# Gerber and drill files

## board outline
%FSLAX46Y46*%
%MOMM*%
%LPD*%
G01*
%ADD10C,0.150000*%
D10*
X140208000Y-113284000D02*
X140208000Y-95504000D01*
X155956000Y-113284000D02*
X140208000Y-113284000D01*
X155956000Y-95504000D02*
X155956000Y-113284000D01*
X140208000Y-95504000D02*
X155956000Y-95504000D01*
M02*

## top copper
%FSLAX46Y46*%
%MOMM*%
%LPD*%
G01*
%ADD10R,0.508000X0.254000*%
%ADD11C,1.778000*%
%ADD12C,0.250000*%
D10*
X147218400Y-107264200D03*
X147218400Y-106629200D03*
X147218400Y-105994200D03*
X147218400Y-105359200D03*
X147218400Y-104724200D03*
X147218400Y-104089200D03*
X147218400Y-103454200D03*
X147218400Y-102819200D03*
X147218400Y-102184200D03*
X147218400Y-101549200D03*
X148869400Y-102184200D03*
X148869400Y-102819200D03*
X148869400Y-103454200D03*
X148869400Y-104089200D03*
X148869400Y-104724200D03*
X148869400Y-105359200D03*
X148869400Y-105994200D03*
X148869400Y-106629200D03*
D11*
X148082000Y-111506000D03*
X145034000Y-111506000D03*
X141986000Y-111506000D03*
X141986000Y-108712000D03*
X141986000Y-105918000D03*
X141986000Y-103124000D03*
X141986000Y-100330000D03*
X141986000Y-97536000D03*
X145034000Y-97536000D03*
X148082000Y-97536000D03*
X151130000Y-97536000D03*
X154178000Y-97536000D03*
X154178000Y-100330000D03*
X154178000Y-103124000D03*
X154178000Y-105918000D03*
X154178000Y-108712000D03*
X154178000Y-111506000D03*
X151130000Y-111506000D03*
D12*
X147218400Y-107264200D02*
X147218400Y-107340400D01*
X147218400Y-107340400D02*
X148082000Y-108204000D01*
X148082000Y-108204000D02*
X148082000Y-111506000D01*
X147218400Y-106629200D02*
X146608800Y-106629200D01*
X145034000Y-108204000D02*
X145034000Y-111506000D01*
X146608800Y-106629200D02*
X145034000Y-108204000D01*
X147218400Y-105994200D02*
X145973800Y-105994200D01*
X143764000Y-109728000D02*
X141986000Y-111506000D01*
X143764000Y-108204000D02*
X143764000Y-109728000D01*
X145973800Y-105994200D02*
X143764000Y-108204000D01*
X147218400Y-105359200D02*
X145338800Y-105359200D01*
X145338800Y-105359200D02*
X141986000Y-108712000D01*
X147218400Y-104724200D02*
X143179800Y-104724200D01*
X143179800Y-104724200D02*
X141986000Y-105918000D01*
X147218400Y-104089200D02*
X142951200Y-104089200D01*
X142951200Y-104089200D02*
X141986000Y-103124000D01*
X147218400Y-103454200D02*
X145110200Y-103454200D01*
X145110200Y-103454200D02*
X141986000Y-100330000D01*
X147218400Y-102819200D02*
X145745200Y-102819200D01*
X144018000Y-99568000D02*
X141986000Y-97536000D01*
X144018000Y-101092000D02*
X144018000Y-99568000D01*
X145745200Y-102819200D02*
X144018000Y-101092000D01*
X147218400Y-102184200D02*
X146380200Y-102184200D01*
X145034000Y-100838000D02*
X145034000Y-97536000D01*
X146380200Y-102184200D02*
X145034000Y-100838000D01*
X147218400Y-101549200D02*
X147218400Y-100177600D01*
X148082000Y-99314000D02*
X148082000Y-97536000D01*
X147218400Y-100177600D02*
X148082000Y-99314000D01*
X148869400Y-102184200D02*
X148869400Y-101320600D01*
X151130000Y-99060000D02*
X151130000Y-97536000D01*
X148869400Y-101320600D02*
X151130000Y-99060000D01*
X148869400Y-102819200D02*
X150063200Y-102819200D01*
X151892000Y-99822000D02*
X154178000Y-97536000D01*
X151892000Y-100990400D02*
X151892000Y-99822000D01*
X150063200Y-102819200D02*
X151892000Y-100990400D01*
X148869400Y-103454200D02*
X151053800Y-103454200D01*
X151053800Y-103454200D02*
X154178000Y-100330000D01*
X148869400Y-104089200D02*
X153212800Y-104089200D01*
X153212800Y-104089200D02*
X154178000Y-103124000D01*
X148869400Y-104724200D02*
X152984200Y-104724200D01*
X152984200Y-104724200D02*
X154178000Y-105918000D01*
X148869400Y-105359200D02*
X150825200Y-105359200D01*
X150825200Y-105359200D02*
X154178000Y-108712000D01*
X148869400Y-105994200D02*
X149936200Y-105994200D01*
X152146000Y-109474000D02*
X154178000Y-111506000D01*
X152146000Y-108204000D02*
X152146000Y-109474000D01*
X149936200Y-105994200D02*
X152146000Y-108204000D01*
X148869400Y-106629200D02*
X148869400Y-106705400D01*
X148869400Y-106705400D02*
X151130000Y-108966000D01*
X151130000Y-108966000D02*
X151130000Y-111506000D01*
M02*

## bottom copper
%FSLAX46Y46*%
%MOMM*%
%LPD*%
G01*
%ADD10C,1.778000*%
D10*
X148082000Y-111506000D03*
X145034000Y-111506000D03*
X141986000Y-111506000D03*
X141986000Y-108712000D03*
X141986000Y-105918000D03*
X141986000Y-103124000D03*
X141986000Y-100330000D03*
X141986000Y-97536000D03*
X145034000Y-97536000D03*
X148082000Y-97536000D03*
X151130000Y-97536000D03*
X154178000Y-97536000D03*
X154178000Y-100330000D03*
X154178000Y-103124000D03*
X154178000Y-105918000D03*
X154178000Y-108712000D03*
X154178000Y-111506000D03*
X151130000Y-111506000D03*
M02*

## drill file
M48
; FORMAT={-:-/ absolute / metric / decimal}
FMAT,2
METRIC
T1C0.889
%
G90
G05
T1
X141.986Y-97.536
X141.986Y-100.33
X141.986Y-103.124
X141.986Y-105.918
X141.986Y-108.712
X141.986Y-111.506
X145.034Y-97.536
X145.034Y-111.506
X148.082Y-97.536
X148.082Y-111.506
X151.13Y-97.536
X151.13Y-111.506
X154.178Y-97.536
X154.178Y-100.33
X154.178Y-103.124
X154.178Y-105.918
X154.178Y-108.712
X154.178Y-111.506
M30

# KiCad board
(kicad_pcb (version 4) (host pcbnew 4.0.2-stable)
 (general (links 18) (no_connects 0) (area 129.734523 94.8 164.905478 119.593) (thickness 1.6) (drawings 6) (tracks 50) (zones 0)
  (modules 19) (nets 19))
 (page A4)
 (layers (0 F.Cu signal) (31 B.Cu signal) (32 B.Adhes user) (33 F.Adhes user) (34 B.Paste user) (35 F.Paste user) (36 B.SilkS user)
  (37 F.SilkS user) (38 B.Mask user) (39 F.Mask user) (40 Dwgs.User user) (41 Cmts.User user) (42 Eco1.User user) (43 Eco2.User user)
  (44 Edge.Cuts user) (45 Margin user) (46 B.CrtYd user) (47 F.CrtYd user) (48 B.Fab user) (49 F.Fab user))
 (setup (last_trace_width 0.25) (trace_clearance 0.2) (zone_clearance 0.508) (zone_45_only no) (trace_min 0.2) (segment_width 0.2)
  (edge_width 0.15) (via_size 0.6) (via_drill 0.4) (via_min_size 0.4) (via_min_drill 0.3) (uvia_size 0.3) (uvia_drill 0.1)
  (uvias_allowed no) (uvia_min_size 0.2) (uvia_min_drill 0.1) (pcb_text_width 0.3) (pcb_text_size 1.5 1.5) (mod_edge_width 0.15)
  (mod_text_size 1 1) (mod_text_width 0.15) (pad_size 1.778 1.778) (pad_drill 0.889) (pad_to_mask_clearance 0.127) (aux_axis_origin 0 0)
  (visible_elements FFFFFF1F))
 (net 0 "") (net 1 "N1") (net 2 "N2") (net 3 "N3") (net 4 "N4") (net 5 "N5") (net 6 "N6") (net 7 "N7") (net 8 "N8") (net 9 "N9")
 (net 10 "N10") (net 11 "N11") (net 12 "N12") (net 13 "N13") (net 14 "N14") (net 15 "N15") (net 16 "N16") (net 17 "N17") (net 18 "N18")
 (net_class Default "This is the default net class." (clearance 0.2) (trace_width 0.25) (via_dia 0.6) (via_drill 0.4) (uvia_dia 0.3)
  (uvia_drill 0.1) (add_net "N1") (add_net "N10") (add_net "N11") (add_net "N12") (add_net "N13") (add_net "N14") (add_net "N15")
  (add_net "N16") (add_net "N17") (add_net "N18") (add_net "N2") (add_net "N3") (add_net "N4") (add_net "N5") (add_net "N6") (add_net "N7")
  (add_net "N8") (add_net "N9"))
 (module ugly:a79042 (layer F.Cu) (at 148.082 104.394)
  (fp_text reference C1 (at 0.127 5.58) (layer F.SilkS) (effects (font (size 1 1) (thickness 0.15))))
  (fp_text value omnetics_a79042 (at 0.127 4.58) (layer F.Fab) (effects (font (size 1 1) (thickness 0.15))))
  (pad 1 smd rect (at -0.8636 2.8702) (size 0.508 0.254) (layers F.Cu F.Paste F.Mask) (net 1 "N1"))
  (pad 2 smd rect (at -0.8636 2.2352) (size 0.508 0.254) (layers F.Cu F.Paste F.Mask) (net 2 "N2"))
  (pad 3 smd rect (at -0.8636 1.6002) (size 0.508 0.254) (layers F.Cu F.Paste F.Mask) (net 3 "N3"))
  (pad 4 smd rect (at -0.8636 0.9652) (size 0.508 0.254) (layers F.Cu F.Paste F.Mask) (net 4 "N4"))
  (pad 5 smd rect (at -0.8636 0.3302) (size 0.508 0.254) (layers F.Cu F.Paste F.Mask) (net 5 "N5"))
  (pad 6 smd rect (at -0.8636 -0.3048) (size 0.508 0.254) (layers F.Cu F.Paste F.Mask) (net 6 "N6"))
  (pad 7 smd rect (at -0.8636 -0.9398) (size 0.508 0.254) (layers F.Cu F.Paste F.Mask) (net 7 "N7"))
  (pad 8 smd rect (at -0.8636 -1.5748) (size 0.508 0.254) (layers F.Cu F.Paste F.Mask) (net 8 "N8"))
  (pad 9 smd rect (at -0.8636 -2.2098) (size 0.508 0.254) (layers F.Cu F.Paste F.Mask) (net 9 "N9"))
  (pad 10 smd rect (at -0.8636 -2.8448) (size 0.508 0.254) (layers F.Cu F.Paste F.Mask) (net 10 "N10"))
  (pad 11 smd rect (at 0.7874 -2.2098) (size 0.508 0.254) (layers F.Cu F.Paste F.Mask) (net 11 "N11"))
  (pad 12 smd rect (at 0.7874 -1.5748) (size 0.508 0.254) (layers F.Cu F.Paste F.Mask) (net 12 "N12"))
  (pad 13 smd rect (at 0.7874 -0.9398) (size 0.508 0.254) (layers F.Cu F.Paste F.Mask) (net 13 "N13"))
  (pad 14 smd rect (at 0.7874 -0.3048) (size 0.508 0.254) (layers F.Cu F.Paste F.Mask) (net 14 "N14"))
  (pad 15 smd rect (at 0.7874 0.3302) (size 0.508 0.254) (layers F.Cu F.Paste F.Mask) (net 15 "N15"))
  (pad 16 smd rect (at 0.7874 0.9652) (size 0.508 0.254) (layers F.Cu F.Paste F.Mask) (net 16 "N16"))
  (pad 17 smd rect (at 0.7874 1.6002) (size 0.508 0.254) (layers F.Cu F.Paste F.Mask) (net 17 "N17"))
  (pad 18 smd rect (at 0.7874 2.2352) (size 0.508 0.254) (layers F.Cu F.Paste F.Mask) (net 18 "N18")))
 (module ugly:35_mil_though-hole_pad (layer F.Cu) (at 147.32 114.3)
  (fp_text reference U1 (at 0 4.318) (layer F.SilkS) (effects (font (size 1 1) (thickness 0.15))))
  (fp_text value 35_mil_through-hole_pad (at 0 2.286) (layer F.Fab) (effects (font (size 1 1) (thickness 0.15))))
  (pad 1 thru_hole circle (at 0.762 -2.794) (size 1.778 1.778) (drill 0.889) (layers *.Cu *.Mask F.SilkS) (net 1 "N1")))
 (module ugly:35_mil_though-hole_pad (layer F.Cu) (at 143.51 114.3)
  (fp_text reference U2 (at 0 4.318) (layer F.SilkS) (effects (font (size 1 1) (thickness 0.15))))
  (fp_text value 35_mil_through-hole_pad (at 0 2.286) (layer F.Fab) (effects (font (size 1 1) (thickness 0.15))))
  (pad 1 thru_hole circle (at 1.524 -2.794) (size 1.778 1.778) (drill 0.889) (layers *.Cu *.Mask F.SilkS) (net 2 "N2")))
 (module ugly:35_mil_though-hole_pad (layer F.Cu) (at 139.7 114.3)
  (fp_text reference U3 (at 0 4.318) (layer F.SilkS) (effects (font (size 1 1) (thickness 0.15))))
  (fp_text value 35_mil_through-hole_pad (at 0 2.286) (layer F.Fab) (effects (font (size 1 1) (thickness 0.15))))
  (pad 1 thru_hole circle (at 2.286 -2.794) (size 1.778 1.778) (drill 0.889) (layers *.Cu *.Mask F.SilkS) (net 3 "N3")))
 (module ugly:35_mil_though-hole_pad (layer F.Cu) (at 139.7 110.49)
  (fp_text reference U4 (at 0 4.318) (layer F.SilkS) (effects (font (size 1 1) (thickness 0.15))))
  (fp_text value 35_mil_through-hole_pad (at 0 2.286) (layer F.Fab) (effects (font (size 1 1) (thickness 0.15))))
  (pad 1 thru_hole circle (at 2.286 -1.778) (size 1.778 1.778) (drill 0.889) (layers *.Cu *.Mask F.SilkS) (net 4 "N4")))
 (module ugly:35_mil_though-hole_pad (layer F.Cu) (at 139.7 106.68)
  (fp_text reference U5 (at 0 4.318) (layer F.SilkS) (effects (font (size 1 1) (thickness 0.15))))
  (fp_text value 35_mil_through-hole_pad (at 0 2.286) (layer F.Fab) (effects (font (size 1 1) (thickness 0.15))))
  (pad 1 thru_hole circle (at 2.286 -0.762) (size 1.778 1.778) (drill 0.889) (layers *.Cu *.Mask F.SilkS) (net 5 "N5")))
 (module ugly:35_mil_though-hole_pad (layer F.Cu) (at 139.7 102.87)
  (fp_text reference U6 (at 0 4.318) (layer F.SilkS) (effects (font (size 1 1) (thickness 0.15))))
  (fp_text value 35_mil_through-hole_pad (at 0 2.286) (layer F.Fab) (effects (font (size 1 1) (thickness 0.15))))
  (pad 1 thru_hole circle (at 2.286 0.254) (size 1.778 1.778) (drill 0.889) (layers *.Cu *.Mask F.SilkS) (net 6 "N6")))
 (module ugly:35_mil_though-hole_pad (layer F.Cu) (at 139.7 99.06)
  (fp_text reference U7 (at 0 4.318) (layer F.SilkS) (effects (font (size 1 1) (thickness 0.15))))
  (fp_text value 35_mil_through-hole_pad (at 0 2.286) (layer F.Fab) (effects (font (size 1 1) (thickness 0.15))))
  (pad 1 thru_hole circle (at 2.286 1.27) (size 1.778 1.778) (drill 0.889) (layers *.Cu *.Mask F.SilkS) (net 7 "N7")))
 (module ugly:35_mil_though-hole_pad (layer F.Cu) (at 139.7 95.25)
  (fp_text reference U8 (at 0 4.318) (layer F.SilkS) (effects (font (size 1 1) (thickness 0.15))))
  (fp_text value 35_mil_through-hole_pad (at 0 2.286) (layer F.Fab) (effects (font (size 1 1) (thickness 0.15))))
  (pad 1 thru_hole circle (at 2.286 2.286) (size 1.778 1.778) (drill 0.889) (layers *.Cu *.Mask F.SilkS) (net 8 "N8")))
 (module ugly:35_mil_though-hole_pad (layer F.Cu) (at 143.51 95.25)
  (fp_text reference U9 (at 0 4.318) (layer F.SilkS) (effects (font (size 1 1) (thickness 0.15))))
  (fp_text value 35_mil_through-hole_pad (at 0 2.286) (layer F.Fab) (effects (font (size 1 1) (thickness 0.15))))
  (pad 1 thru_hole circle (at 1.524 2.286) (size 1.778 1.778) (drill 0.889) (layers *.Cu *.Mask F.SilkS) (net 9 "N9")))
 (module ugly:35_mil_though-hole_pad (layer F.Cu) (at 147.32 95.25)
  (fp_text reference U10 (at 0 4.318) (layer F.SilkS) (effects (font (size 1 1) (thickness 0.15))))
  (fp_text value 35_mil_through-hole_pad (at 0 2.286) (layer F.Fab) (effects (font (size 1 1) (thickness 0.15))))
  (pad 1 thru_hole circle (at 0.762 2.286) (size 1.778 1.778) (drill 0.889) (layers *.Cu *.Mask F.SilkS) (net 10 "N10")))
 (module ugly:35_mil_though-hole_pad (layer F.Cu) (at 151.13 95.25)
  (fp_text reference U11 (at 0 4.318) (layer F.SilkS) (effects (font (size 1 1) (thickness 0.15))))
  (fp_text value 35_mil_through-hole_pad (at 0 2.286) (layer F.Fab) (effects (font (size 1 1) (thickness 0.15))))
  (pad 1 thru_hole circle (at 0 2.286) (size 1.778 1.778) (drill 0.889) (layers *.Cu *.Mask F.SilkS) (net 11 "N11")))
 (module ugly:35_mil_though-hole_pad (layer F.Cu) (at 154.94 95.25)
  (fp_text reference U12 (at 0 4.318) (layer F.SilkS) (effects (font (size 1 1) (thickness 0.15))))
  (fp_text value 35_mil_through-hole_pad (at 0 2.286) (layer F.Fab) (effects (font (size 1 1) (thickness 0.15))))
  (pad 1 thru_hole circle (at -0.762 2.286) (size 1.778 1.778) (drill 0.889) (layers *.Cu *.Mask F.SilkS) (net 12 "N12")))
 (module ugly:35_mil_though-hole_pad (layer F.Cu) (at 154.94 99.06)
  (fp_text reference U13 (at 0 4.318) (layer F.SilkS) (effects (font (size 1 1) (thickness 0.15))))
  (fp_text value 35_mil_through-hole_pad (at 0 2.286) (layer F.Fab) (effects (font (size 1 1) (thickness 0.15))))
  (pad 1 thru_hole circle (at -0.762 1.27) (size 1.778 1.778) (drill 0.889) (layers *.Cu *.Mask F.SilkS) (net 13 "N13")))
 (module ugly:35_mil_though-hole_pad (layer F.Cu) (at 154.94 102.87)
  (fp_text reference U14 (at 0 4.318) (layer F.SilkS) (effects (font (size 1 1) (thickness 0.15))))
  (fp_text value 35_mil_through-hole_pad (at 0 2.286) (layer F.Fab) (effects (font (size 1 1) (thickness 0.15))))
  (pad 1 thru_hole circle (at -0.762 0.254) (size 1.778 1.778) (drill 0.889) (layers *.Cu *.Mask F.SilkS) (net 14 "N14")))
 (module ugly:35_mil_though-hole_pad (layer F.Cu) (at 154.94 106.68)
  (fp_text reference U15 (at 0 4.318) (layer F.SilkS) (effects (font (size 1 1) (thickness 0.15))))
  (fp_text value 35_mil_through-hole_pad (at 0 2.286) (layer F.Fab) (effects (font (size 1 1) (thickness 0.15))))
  (pad 1 thru_hole circle (at -0.762 -0.762) (size 1.778 1.778) (drill 0.889) (layers *.Cu *.Mask F.SilkS) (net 15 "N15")))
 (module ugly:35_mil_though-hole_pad (layer F.Cu) (at 154.94 110.49)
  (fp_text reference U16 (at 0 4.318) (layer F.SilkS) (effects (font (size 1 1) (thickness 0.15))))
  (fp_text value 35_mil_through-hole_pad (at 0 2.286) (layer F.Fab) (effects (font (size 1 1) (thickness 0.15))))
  (pad 1 thru_hole circle (at -0.762 -1.778) (size 1.778 1.778) (drill 0.889) (layers *.Cu *.Mask F.SilkS) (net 16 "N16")))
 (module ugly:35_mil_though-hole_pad (layer F.Cu) (at 154.94 114.3)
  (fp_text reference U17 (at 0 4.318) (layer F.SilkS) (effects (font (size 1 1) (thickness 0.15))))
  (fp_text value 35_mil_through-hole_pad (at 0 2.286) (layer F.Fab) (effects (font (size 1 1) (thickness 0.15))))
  (pad 1 thru_hole circle (at -0.762 -2.794) (size 1.778 1.778) (drill 0.889) (layers *.Cu *.Mask F.SilkS) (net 17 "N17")))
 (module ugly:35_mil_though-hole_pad (layer F.Cu) (at 151.13 114.046)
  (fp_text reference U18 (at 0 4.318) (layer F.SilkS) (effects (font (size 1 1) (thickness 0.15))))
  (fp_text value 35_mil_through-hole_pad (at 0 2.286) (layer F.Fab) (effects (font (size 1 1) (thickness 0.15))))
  (pad 1 thru_hole circle (at 0 -2.54) (size 1.778 1.778) (drill 0.889) (layers *.Cu *.Mask F.SilkS) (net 18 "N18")))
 (gr_line (start 140.208 113.284) (end 140.208 95.504) (angle 90) (layer Edge.Cuts) (width 0.15))
 (gr_line (start 155.956 113.284) (end 140.208 113.284) (angle 90) (layer Edge.Cuts) (width 0.15))
 (gr_line (start 155.956 95.504) (end 155.956 113.284) (angle 90) (layer Edge.Cuts) (width 0.15))
 (gr_line (start 140.208 95.504) (end 155.956 95.504) (angle 90) (layer Edge.Cuts) (width 0.15))
 (segment (start 147.2184 107.2642) (end 147.2184 107.3404) (width 0.25) (layer F.Cu) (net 1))
 (segment (start 147.2184 107.3404) (end 148.082 108.204) (width 0.25) (layer F.Cu) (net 1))
 (segment (start 148.082 108.204) (end 148.082 111.506) (width 0.25) (layer F.Cu) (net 1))
 (segment (start 147.2184 106.6292) (end 146.6088 106.6292) (width 0.25) (layer F.Cu) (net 2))
 (segment (start 145.034 108.204) (end 145.034 111.506) (width 0.25) (layer F.Cu) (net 2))
 (segment (start 146.6088 106.6292) (end 145.034 108.204) (width 0.25) (layer F.Cu) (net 2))
 (segment (start 147.2184 105.9942) (end 145.9738 105.9942) (width 0.25) (layer F.Cu) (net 3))
 (segment (start 143.764 109.728) (end 141.986 111.506) (width 0.25) (layer F.Cu) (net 3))
 (segment (start 143.764 108.204) (end 143.764 109.728) (width 0.25) (layer F.Cu) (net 3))
 (segment (start 145.9738 105.9942) (end 143.764 108.204) (width 0.25) (layer F.Cu) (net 3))
 (segment (start 147.2184 105.3592) (end 145.3388 105.3592) (width 0.25) (layer F.Cu) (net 4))
 (segment (start 145.3388 105.3592) (end 141.986 108.712) (width 0.25) (layer F.Cu) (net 4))
 (segment (start 147.2184 104.7242) (end 143.1798 104.7242) (width 0.25) (layer F.Cu) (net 5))
 (segment (start 143.1798 104.7242) (end 141.986 105.918) (width 0.25) (layer F.Cu) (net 5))
 (segment (start 147.2184 104.0892) (end 142.9512 104.0892) (width 0.25) (layer F.Cu) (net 6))
 (segment (start 142.9512 104.0892) (end 141.986 103.124) (width 0.25) (layer F.Cu) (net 6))
 (segment (start 147.2184 103.4542) (end 145.1102 103.4542) (width 0.25) (layer F.Cu) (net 7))
 (segment (start 145.1102 103.4542) (end 141.986 100.33) (width 0.25) (layer F.Cu) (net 7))
 (segment (start 147.2184 102.8192) (end 145.7452 102.8192) (width 0.25) (layer F.Cu) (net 8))
 (segment (start 144.018 99.568) (end 141.986 97.536) (width 0.25) (layer F.Cu) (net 8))
 (segment (start 144.018 101.092) (end 144.018 99.568) (width 0.25) (layer F.Cu) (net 8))
 (segment (start 145.7452 102.8192) (end 144.018 101.092) (width 0.25) (layer F.Cu) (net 8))
 (segment (start 147.2184 102.1842) (end 146.3802 102.1842) (width 0.25) (layer F.Cu) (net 9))
 (segment (start 145.034 100.838) (end 145.034 97.536) (width 0.25) (layer F.Cu) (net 9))
 (segment (start 146.3802 102.1842) (end 145.034 100.838) (width 0.25) (layer F.Cu) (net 9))
 (segment (start 147.2184 101.5492) (end 147.2184 100.1776) (width 0.25) (layer F.Cu) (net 10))
 (segment (start 148.082 99.314) (end 148.082 97.536) (width 0.25) (layer F.Cu) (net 10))
 (segment (start 147.2184 100.1776) (end 148.082 99.314) (width 0.25) (layer F.Cu) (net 10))
 (segment (start 148.8694 102.1842) (end 148.8694 101.3206) (width 0.25) (layer F.Cu) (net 11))
 (segment (start 151.13 99.06) (end 151.13 97.536) (width 0.25) (layer F.Cu) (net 11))
 (segment (start 148.8694 101.3206) (end 151.13 99.06) (width 0.25) (layer F.Cu) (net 11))
 (segment (start 148.8694 102.8192) (end 150.0632 102.8192) (width 0.25) (layer F.Cu) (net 12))
 (segment (start 151.892 99.822) (end 154.178 97.536) (width 0.25) (layer F.Cu) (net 12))
 (segment (start 151.892 100.9904) (end 151.892 99.822) (width 0.25) (layer F.Cu) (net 12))
 (segment (start 150.0632 102.8192) (end 151.892 100.9904) (width 0.25) (layer F.Cu) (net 12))
 (segment (start 148.8694 103.4542) (end 151.0538 103.4542) (width 0.25) (layer F.Cu) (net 13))
 (segment (start 151.0538 103.4542) (end 154.178 100.33) (width 0.25) (layer F.Cu) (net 13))
 (segment (start 148.8694 104.0892) (end 153.2128 104.0892) (width 0.25) (layer F.Cu) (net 14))
 (segment (start 153.2128 104.0892) (end 154.178 103.124) (width 0.25) (layer F.Cu) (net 14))
 (segment (start 148.8694 104.7242) (end 152.9842 104.7242) (width 0.25) (layer F.Cu) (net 15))
 (segment (start 152.9842 104.7242) (end 154.178 105.918) (width 0.25) (layer F.Cu) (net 15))
 (segment (start 148.8694 105.3592) (end 150.8252 105.3592) (width 0.25) (layer F.Cu) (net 16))
 (segment (start 150.8252 105.3592) (end 154.178 108.712) (width 0.25) (layer F.Cu) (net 16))
 (segment (start 148.8694 105.9942) (end 149.9362 105.9942) (width 0.25) (layer F.Cu) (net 17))
 (segment (start 152.146 109.474) (end 154.178 111.506) (width 0.25) (layer F.Cu) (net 17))
 (segment (start 152.146 108.204) (end 152.146 109.474) (width 0.25) (layer F.Cu) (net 17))
 (segment (start 149.9362 105.9942) (end 152.146 108.204) (width 0.25) (layer F.Cu) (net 17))
 (segment (start 148.8694 106.6292) (end 148.8694 106.7054) (width 0.25) (layer F.Cu) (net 18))
 (segment (start 148.8694 106.7054) (end 151.13 108.966) (width 0.25) (layer F.Cu) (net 18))
 (segment (start 151.13 108.966) (end 151.13 111.506) (width 0.25) (layer F.Cu) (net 18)))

